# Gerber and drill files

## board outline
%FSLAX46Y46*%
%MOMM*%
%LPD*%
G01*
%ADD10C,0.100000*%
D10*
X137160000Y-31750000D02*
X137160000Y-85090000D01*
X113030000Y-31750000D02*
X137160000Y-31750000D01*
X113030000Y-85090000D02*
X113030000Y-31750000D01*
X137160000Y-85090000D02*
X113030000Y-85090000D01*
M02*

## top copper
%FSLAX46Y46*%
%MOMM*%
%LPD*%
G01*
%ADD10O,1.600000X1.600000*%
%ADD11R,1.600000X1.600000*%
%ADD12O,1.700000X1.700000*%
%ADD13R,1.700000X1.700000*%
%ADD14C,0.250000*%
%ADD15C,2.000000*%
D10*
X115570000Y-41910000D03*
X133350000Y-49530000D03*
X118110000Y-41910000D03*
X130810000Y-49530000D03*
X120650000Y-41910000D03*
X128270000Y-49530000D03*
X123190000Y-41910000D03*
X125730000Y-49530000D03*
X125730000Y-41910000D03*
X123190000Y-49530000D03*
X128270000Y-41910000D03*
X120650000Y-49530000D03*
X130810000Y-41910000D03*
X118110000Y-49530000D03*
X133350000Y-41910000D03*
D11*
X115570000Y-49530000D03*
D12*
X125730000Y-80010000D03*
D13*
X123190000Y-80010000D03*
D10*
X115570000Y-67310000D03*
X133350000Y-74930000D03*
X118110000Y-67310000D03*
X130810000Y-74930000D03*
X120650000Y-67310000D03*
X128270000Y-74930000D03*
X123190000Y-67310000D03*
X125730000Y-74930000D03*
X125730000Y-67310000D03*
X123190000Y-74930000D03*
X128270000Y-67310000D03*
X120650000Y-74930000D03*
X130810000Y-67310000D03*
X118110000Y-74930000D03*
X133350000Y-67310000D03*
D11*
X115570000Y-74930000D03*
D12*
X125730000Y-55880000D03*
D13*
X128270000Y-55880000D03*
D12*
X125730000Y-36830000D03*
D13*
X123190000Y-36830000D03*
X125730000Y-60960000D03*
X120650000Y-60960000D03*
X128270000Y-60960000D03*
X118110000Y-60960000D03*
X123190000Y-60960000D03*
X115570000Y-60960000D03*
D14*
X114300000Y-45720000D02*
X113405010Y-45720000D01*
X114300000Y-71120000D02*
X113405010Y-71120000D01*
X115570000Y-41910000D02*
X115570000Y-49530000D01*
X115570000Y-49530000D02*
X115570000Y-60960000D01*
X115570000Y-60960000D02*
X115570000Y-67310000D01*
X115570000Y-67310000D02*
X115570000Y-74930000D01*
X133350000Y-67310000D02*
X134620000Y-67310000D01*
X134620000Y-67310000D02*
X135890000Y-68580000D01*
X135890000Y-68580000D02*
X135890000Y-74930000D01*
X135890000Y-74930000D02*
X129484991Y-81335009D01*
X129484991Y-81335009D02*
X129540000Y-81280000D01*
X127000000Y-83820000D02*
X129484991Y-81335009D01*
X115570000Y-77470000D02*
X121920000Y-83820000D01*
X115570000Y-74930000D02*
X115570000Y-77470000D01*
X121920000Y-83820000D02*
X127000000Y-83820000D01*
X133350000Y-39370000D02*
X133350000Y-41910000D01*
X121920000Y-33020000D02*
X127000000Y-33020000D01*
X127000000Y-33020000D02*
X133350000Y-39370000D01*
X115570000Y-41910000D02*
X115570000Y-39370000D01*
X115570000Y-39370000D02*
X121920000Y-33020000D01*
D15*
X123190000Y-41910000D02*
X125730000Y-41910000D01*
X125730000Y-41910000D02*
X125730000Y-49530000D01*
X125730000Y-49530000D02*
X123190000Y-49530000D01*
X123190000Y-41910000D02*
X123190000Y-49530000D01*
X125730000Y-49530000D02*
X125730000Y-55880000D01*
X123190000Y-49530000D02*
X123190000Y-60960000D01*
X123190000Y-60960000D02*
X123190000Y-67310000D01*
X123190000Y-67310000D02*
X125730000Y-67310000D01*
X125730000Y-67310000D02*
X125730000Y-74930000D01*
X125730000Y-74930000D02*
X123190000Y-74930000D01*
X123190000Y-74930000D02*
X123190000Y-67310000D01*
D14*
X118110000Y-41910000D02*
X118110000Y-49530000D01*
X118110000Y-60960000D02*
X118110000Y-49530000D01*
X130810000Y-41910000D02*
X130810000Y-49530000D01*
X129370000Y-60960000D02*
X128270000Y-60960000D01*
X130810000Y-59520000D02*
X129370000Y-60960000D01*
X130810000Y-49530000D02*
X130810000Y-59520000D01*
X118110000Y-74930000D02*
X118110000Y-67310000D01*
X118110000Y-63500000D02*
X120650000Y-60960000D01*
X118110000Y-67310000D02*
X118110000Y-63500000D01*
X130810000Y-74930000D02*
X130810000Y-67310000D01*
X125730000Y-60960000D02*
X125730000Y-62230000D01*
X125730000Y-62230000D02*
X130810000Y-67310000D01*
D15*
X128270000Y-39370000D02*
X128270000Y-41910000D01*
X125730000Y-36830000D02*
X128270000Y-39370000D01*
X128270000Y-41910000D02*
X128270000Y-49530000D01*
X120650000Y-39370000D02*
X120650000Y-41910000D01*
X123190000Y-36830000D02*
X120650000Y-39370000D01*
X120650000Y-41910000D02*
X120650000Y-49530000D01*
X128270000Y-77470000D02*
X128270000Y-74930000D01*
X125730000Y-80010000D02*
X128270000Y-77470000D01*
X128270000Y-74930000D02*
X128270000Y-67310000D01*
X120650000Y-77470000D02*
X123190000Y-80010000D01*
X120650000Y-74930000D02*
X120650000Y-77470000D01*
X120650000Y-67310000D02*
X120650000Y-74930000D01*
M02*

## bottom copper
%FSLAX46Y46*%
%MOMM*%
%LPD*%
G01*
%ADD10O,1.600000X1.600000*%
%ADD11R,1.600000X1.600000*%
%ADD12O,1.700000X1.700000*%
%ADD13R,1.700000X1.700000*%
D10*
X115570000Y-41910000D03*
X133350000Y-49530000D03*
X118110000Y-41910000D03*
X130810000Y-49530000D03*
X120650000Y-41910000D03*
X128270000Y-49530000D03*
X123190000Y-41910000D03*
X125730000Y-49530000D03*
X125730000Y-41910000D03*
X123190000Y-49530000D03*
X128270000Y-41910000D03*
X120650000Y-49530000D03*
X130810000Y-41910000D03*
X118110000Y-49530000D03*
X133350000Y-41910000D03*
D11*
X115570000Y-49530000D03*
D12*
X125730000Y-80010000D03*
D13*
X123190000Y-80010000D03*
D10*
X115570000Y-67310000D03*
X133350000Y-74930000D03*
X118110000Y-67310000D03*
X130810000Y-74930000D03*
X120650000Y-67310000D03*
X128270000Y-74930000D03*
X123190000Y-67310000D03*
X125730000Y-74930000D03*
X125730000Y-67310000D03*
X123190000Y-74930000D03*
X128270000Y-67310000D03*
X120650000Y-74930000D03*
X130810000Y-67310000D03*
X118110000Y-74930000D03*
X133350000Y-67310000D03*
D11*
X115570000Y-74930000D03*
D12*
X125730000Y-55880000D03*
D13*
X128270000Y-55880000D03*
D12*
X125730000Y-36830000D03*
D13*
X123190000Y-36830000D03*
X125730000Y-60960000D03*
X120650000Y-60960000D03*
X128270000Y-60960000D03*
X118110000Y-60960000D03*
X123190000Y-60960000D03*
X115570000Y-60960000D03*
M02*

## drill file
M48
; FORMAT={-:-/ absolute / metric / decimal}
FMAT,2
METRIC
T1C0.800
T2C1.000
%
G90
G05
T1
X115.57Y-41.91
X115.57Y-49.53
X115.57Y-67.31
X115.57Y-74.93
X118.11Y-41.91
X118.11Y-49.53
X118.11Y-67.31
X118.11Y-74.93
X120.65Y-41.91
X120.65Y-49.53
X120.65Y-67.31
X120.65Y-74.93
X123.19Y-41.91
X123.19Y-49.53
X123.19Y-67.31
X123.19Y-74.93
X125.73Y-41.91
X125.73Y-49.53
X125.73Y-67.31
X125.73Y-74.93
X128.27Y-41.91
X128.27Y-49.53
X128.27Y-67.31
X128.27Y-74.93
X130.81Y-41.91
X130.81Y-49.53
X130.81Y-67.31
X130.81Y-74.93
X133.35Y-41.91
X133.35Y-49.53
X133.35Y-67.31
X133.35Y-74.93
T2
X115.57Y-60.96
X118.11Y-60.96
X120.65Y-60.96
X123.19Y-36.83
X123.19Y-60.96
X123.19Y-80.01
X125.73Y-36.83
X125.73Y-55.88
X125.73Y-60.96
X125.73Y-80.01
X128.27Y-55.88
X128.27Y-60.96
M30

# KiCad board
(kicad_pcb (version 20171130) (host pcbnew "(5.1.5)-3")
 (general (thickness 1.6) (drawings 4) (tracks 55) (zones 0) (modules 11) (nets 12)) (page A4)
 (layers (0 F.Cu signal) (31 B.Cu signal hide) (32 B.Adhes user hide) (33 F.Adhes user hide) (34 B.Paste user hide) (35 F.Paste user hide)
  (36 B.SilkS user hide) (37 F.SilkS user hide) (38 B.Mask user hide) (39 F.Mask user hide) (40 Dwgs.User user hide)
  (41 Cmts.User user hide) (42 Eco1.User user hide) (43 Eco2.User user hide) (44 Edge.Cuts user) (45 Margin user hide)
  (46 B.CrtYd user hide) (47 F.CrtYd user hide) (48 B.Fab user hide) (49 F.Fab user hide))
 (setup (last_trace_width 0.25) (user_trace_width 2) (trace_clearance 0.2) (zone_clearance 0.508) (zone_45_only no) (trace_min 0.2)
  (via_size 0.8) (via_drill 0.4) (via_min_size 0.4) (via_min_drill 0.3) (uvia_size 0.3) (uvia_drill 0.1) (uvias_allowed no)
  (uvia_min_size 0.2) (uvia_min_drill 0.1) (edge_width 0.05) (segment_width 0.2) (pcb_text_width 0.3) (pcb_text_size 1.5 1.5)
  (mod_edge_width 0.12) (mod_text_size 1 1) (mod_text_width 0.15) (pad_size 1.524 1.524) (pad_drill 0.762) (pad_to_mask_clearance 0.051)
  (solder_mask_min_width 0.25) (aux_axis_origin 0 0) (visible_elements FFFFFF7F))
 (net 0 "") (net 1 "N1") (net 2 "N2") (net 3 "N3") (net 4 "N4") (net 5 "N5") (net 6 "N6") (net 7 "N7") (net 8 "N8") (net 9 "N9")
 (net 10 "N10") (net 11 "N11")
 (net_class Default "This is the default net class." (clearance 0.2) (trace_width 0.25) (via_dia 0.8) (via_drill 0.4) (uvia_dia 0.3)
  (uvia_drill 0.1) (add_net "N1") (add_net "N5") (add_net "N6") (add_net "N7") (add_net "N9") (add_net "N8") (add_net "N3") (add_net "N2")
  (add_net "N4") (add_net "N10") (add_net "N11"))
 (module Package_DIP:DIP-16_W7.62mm (layer F.Cu) (at 115.57 49.53 90)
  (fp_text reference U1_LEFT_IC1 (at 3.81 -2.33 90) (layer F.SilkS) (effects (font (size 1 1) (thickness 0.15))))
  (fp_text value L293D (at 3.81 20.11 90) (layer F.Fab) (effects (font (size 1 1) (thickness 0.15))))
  (pad 16 thru_hole oval (at 7.62 0 90) (size 1.6 1.6) (drill 0.8) (layers *.Cu *.Mask) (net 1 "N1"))
  (pad 8 thru_hole oval (at 0 17.78 90) (size 1.6 1.6) (drill 0.8) (layers *.Cu *.Mask) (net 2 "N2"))
  (pad 15 thru_hole oval (at 7.62 2.54 90) (size 1.6 1.6) (drill 0.8) (layers *.Cu *.Mask) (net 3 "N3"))
  (pad 7 thru_hole oval (at 0 15.24 90) (size 1.6 1.6) (drill 0.8) (layers *.Cu *.Mask) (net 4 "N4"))
  (pad 14 thru_hole oval (at 7.62 5.08 90) (size 1.6 1.6) (drill 0.8) (layers *.Cu *.Mask) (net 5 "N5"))
  (pad 6 thru_hole oval (at 0 12.7 90) (size 1.6 1.6) (drill 0.8) (layers *.Cu *.Mask) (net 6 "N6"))
  (pad 13 thru_hole oval (at 7.62 7.62 90) (size 1.6 1.6) (drill 0.8) (layers *.Cu *.Mask) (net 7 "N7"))
  (pad 5 thru_hole oval (at 0 10.16 90) (size 1.6 1.6) (drill 0.8) (layers *.Cu *.Mask) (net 7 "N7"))
  (pad 12 thru_hole oval (at 7.62 10.16 90) (size 1.6 1.6) (drill 0.8) (layers *.Cu *.Mask) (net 7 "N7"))
  (pad 4 thru_hole oval (at 0 7.62 90) (size 1.6 1.6) (drill 0.8) (layers *.Cu *.Mask) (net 7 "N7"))
  (pad 11 thru_hole oval (at 7.62 12.7 90) (size 1.6 1.6) (drill 0.8) (layers *.Cu *.Mask) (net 6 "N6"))
  (pad 3 thru_hole oval (at 0 5.08 90) (size 1.6 1.6) (drill 0.8) (layers *.Cu *.Mask) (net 5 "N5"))
  (pad 10 thru_hole oval (at 7.62 15.24 90) (size 1.6 1.6) (drill 0.8) (layers *.Cu *.Mask) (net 4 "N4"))
  (pad 2 thru_hole oval (at 0 2.54 90) (size 1.6 1.6) (drill 0.8) (layers *.Cu *.Mask) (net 3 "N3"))
  (pad 9 thru_hole oval (at 7.62 17.78 90) (size 1.6 1.6) (drill 0.8) (layers *.Cu *.Mask) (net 1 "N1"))
  (pad 1 thru_hole rect (at 0 0 90) (size 1.6 1.6) (drill 0.8) (layers *.Cu *.Mask) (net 1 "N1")))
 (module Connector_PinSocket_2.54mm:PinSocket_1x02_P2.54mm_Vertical (layer F.Cu) (at 123.19 80.01 90)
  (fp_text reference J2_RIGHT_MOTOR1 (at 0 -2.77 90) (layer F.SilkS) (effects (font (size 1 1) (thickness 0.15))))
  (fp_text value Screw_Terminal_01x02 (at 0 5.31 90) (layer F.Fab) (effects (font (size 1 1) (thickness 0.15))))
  (pad 2 thru_hole oval (at 0 2.54 90) (size 1.7 1.7) (drill 1) (layers *.Cu *.Mask) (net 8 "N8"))
  (pad 1 thru_hole rect (at 0 0 90) (size 1.7 1.7) (drill 1) (layers *.Cu *.Mask) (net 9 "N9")))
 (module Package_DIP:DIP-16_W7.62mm (layer F.Cu) (at 115.57 74.93 90)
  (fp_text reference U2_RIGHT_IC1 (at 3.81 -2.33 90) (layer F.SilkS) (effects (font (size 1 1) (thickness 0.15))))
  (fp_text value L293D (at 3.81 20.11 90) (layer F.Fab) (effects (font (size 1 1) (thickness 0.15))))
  (pad 16 thru_hole oval (at 7.62 0 90) (size 1.6 1.6) (drill 0.8) (layers *.Cu *.Mask) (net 1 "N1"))
  (pad 8 thru_hole oval (at 0 17.78 90) (size 1.6 1.6) (drill 0.8) (layers *.Cu *.Mask) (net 2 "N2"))
  (pad 15 thru_hole oval (at 7.62 2.54 90) (size 1.6 1.6) (drill 0.8) (layers *.Cu *.Mask) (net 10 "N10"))
  (pad 7 thru_hole oval (at 0 15.24 90) (size 1.6 1.6) (drill 0.8) (layers *.Cu *.Mask) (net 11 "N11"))
  (pad 14 thru_hole oval (at 7.62 5.08 90) (size 1.6 1.6) (drill 0.8) (layers *.Cu *.Mask) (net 9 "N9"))
  (pad 6 thru_hole oval (at 0 12.7 90) (size 1.6 1.6) (drill 0.8) (layers *.Cu *.Mask) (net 8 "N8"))
  (pad 13 thru_hole oval (at 7.62 7.62 90) (size 1.6 1.6) (drill 0.8) (layers *.Cu *.Mask) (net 7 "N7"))
  (pad 5 thru_hole oval (at 0 10.16 90) (size 1.6 1.6) (drill 0.8) (layers *.Cu *.Mask) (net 7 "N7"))
  (pad 12 thru_hole oval (at 7.62 10.16 90) (size 1.6 1.6) (drill 0.8) (layers *.Cu *.Mask) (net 7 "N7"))
  (pad 4 thru_hole oval (at 0 7.62 90) (size 1.6 1.6) (drill 0.8) (layers *.Cu *.Mask) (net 7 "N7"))
  (pad 11 thru_hole oval (at 7.62 12.7 90) (size 1.6 1.6) (drill 0.8) (layers *.Cu *.Mask) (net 8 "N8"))
  (pad 3 thru_hole oval (at 0 5.08 90) (size 1.6 1.6) (drill 0.8) (layers *.Cu *.Mask) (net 9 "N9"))
  (pad 10 thru_hole oval (at 7.62 15.24 90) (size 1.6 1.6) (drill 0.8) (layers *.Cu *.Mask) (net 11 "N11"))
  (pad 2 thru_hole oval (at 0 2.54 90) (size 1.6 1.6) (drill 0.8) (layers *.Cu *.Mask) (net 10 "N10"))
  (pad 9 thru_hole oval (at 7.62 17.78 90) (size 1.6 1.6) (drill 0.8) (layers *.Cu *.Mask) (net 1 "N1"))
  (pad 1 thru_hole rect (at 0 0 90) (size 1.6 1.6) (drill 0.8) (layers *.Cu *.Mask) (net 1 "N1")))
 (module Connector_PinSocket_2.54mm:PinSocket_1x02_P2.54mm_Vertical (layer F.Cu) (at 128.27 55.88 270)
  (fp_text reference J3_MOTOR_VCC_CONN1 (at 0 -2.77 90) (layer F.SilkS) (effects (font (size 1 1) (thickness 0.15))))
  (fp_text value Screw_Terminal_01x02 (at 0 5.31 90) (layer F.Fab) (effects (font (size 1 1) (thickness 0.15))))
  (pad 2 thru_hole oval (at 0 2.54 270) (size 1.7 1.7) (drill 1) (layers *.Cu *.Mask) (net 7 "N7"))
  (pad 1 thru_hole rect (at 0 0 270) (size 1.7 1.7) (drill 1) (layers *.Cu *.Mask) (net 2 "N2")))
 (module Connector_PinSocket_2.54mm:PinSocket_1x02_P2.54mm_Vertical (layer F.Cu) (at 123.19 36.83 90)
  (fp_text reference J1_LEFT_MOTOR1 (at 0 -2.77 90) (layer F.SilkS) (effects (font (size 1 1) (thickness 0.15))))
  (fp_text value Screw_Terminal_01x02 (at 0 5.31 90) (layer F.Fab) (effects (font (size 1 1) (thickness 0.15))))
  (pad 2 thru_hole oval (at 0 2.54 90) (size 1.7 1.7) (drill 1) (layers *.Cu *.Mask) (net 6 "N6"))
  (pad 1 thru_hole rect (at 0 0 90) (size 1.7 1.7) (drill 1) (layers *.Cu *.Mask) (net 5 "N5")))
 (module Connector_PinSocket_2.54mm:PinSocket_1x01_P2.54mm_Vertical (layer F.Cu) (at 125.73 60.96)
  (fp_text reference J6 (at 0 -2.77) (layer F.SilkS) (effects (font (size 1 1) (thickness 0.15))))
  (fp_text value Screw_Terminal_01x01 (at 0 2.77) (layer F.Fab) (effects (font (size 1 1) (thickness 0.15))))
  (pad 1 thru_hole rect (at 0 0) (size 1.7 1.7) (drill 1) (layers *.Cu *.Mask) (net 11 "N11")))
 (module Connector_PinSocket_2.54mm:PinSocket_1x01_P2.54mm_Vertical (layer F.Cu) (at 120.65 60.96)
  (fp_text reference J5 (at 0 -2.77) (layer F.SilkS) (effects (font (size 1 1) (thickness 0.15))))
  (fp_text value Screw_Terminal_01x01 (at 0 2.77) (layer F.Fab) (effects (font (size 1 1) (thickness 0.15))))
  (pad 1 thru_hole rect (at 0 0) (size 1.7 1.7) (drill 1) (layers *.Cu *.Mask) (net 10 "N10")))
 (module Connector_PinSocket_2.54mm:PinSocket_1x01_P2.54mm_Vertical (layer F.Cu) (at 128.27 60.96)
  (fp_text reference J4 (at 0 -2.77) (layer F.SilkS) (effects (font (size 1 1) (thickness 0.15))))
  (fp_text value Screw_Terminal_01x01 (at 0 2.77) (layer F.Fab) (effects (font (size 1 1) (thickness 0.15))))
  (pad 1 thru_hole rect (at 0 0) (size 1.7 1.7) (drill 1) (layers *.Cu *.Mask) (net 4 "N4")))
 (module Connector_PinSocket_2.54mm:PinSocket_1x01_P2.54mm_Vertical (layer F.Cu) (at 118.11 60.96)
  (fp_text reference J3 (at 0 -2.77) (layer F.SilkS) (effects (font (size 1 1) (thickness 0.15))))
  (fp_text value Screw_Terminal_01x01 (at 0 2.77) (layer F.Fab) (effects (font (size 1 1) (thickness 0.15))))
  (pad 1 thru_hole rect (at 0 0) (size 1.7 1.7) (drill 1) (layers *.Cu *.Mask) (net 3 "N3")))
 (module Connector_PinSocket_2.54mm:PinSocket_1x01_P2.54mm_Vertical (layer F.Cu) (at 123.19 60.96)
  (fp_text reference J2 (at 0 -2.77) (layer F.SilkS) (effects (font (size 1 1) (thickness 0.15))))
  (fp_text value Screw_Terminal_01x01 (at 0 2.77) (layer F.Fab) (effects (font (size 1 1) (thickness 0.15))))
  (pad 1 thru_hole rect (at 0 0) (size 1.7 1.7) (drill 1) (layers *.Cu *.Mask) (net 7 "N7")))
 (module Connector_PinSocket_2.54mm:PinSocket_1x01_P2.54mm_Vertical (layer F.Cu) (at 115.57 60.96)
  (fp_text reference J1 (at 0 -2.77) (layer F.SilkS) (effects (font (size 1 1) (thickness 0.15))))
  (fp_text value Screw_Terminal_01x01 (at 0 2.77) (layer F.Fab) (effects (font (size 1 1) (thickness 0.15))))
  (pad 1 thru_hole rect (at 0 0) (size 1.7 1.7) (drill 1) (layers *.Cu *.Mask) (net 1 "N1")))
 (gr_line (start 137.16 31.75) (end 137.16 85.09) (layer Edge.Cuts) (width 0.1))
 (gr_line (start 113.03 31.75) (end 137.16 31.75) (layer Edge.Cuts) (width 0.1))
 (gr_line (start 113.03 85.09) (end 113.03 31.75) (layer Edge.Cuts) (width 0.1))
 (gr_line (start 137.16 85.09) (end 113.03 85.09) (layer Edge.Cuts) (width 0.1))
 (segment (start 114.3 45.72) (end 113.40501 45.72) (width 0.25) (layer F.Cu) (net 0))
 (segment (start 114.3 71.12) (end 113.40501 71.12) (width 0.25) (layer F.Cu) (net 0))
 (segment (start 115.57 41.91) (end 115.57 49.53) (width 0.25) (layer F.Cu) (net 1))
 (segment (start 115.57 49.53) (end 115.57 60.96) (width 0.25) (layer F.Cu) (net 1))
 (segment (start 115.57 60.96) (end 115.57 67.31) (width 0.25) (layer F.Cu) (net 1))
 (segment (start 115.57 67.31) (end 115.57 74.93) (width 0.25) (layer F.Cu) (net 1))
 (segment (start 133.35 67.31) (end 134.62 67.31) (width 0.25) (layer F.Cu) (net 1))
 (segment (start 134.62 67.31) (end 135.89 68.58) (width 0.25) (layer F.Cu) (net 1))
 (segment (start 135.89 68.58) (end 135.89 74.93) (width 0.25) (layer F.Cu) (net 1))
 (segment (start 135.89 74.93) (end 129.484991 81.335009) (width 0.25) (layer F.Cu) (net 1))
 (segment (start 129.484991 81.335009) (end 129.54 81.28) (width 0.25) (layer F.Cu) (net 1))
 (segment (start 127 83.82) (end 129.484991 81.335009) (width 0.25) (layer F.Cu) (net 1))
 (segment (start 115.57 77.47) (end 121.92 83.82) (width 0.25) (layer F.Cu) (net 1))
 (segment (start 115.57 74.93) (end 115.57 77.47) (width 0.25) (layer F.Cu) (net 1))
 (segment (start 121.92 83.82) (end 127 83.82) (width 0.25) (layer F.Cu) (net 1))
 (segment (start 133.35 39.37) (end 133.35 41.91) (width 0.25) (layer F.Cu) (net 1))
 (segment (start 121.92 33.02) (end 127 33.02) (width 0.25) (layer F.Cu) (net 1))
 (segment (start 127 33.02) (end 133.35 39.37) (width 0.25) (layer F.Cu) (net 1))
 (segment (start 115.57 41.91) (end 115.57 39.37) (width 0.25) (layer F.Cu) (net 1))
 (segment (start 115.57 39.37) (end 121.92 33.02) (width 0.25) (layer F.Cu) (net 1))
 (segment (start 123.19 41.91) (end 125.73 41.91) (width 2) (layer F.Cu) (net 7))
 (segment (start 125.73 41.91) (end 125.73 49.53) (width 2) (layer F.Cu) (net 7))
 (segment (start 125.73 49.53) (end 123.19 49.53) (width 2) (layer F.Cu) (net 7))
 (segment (start 123.19 41.91) (end 123.19 49.53) (width 2) (layer F.Cu) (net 7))
 (segment (start 125.73 49.53) (end 125.73 55.88) (width 2) (layer F.Cu) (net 7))
 (segment (start 123.19 49.53) (end 123.19 60.96) (width 2) (layer F.Cu) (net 7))
 (segment (start 123.19 60.96) (end 123.19 67.31) (width 2) (layer F.Cu) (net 7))
 (segment (start 123.19 67.31) (end 125.73 67.31) (width 2) (layer F.Cu) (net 7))
 (segment (start 125.73 67.31) (end 125.73 74.93) (width 2) (layer F.Cu) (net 7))
 (segment (start 125.73 74.93) (end 123.19 74.93) (width 2) (layer F.Cu) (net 7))
 (segment (start 123.19 74.93) (end 123.19 67.31) (width 2) (layer F.Cu) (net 7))
 (segment (start 118.11 41.91) (end 118.11 49.53) (width 0.25) (layer F.Cu) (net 3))
 (segment (start 118.11 60.96) (end 118.11 49.53) (width 0.25) (layer F.Cu) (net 3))
 (segment (start 130.81 41.91) (end 130.81 49.53) (width 0.25) (layer F.Cu) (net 4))
 (segment (start 129.37 60.96) (end 128.27 60.96) (width 0.25) (layer F.Cu) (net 4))
 (segment (start 130.81 59.52) (end 129.37 60.96) (width 0.25) (layer F.Cu) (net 4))
 (segment (start 130.81 49.53) (end 130.81 59.52) (width 0.25) (layer F.Cu) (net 4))
 (segment (start 118.11 74.93) (end 118.11 67.31) (width 0.25) (layer F.Cu) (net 10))
 (segment (start 118.11 63.5) (end 120.65 60.96) (width 0.25) (layer F.Cu) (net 10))
 (segment (start 118.11 67.31) (end 118.11 63.5) (width 0.25) (layer F.Cu) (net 10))
 (segment (start 130.81 74.93) (end 130.81 67.31) (width 0.25) (layer F.Cu) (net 11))
 (segment (start 125.73 60.96) (end 125.73 62.23) (width 0.25) (layer F.Cu) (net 11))
 (segment (start 125.73 62.23) (end 130.81 67.31) (width 0.25) (layer F.Cu) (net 11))
 (segment (start 128.27 39.37) (end 128.27 41.91) (width 2) (layer F.Cu) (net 6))
 (segment (start 125.73 36.83) (end 128.27 39.37) (width 2) (layer F.Cu) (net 6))
 (segment (start 128.27 41.91) (end 128.27 49.53) (width 2) (layer F.Cu) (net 6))
 (segment (start 120.65 39.37) (end 120.65 41.91) (width 2) (layer F.Cu) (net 5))
 (segment (start 123.19 36.83) (end 120.65 39.37) (width 2) (layer F.Cu) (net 5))
 (segment (start 120.65 41.91) (end 120.65 49.53) (width 2) (layer F.Cu) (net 5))
 (segment (start 128.27 77.47) (end 128.27 74.93) (width 2) (layer F.Cu) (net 8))
 (segment (start 125.73 80.01) (end 128.27 77.47) (width 2) (layer F.Cu) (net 8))
 (segment (start 128.27 74.93) (end 128.27 67.31) (width 2) (layer F.Cu) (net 8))
 (segment (start 120.65 77.47) (end 123.19 80.01) (width 2) (layer F.Cu) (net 9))
 (segment (start 120.65 74.93) (end 120.65 77.47) (width 2) (layer F.Cu) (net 9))
 (segment (start 120.65 67.31) (end 120.65 74.93) (width 2) (layer F.Cu) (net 9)))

